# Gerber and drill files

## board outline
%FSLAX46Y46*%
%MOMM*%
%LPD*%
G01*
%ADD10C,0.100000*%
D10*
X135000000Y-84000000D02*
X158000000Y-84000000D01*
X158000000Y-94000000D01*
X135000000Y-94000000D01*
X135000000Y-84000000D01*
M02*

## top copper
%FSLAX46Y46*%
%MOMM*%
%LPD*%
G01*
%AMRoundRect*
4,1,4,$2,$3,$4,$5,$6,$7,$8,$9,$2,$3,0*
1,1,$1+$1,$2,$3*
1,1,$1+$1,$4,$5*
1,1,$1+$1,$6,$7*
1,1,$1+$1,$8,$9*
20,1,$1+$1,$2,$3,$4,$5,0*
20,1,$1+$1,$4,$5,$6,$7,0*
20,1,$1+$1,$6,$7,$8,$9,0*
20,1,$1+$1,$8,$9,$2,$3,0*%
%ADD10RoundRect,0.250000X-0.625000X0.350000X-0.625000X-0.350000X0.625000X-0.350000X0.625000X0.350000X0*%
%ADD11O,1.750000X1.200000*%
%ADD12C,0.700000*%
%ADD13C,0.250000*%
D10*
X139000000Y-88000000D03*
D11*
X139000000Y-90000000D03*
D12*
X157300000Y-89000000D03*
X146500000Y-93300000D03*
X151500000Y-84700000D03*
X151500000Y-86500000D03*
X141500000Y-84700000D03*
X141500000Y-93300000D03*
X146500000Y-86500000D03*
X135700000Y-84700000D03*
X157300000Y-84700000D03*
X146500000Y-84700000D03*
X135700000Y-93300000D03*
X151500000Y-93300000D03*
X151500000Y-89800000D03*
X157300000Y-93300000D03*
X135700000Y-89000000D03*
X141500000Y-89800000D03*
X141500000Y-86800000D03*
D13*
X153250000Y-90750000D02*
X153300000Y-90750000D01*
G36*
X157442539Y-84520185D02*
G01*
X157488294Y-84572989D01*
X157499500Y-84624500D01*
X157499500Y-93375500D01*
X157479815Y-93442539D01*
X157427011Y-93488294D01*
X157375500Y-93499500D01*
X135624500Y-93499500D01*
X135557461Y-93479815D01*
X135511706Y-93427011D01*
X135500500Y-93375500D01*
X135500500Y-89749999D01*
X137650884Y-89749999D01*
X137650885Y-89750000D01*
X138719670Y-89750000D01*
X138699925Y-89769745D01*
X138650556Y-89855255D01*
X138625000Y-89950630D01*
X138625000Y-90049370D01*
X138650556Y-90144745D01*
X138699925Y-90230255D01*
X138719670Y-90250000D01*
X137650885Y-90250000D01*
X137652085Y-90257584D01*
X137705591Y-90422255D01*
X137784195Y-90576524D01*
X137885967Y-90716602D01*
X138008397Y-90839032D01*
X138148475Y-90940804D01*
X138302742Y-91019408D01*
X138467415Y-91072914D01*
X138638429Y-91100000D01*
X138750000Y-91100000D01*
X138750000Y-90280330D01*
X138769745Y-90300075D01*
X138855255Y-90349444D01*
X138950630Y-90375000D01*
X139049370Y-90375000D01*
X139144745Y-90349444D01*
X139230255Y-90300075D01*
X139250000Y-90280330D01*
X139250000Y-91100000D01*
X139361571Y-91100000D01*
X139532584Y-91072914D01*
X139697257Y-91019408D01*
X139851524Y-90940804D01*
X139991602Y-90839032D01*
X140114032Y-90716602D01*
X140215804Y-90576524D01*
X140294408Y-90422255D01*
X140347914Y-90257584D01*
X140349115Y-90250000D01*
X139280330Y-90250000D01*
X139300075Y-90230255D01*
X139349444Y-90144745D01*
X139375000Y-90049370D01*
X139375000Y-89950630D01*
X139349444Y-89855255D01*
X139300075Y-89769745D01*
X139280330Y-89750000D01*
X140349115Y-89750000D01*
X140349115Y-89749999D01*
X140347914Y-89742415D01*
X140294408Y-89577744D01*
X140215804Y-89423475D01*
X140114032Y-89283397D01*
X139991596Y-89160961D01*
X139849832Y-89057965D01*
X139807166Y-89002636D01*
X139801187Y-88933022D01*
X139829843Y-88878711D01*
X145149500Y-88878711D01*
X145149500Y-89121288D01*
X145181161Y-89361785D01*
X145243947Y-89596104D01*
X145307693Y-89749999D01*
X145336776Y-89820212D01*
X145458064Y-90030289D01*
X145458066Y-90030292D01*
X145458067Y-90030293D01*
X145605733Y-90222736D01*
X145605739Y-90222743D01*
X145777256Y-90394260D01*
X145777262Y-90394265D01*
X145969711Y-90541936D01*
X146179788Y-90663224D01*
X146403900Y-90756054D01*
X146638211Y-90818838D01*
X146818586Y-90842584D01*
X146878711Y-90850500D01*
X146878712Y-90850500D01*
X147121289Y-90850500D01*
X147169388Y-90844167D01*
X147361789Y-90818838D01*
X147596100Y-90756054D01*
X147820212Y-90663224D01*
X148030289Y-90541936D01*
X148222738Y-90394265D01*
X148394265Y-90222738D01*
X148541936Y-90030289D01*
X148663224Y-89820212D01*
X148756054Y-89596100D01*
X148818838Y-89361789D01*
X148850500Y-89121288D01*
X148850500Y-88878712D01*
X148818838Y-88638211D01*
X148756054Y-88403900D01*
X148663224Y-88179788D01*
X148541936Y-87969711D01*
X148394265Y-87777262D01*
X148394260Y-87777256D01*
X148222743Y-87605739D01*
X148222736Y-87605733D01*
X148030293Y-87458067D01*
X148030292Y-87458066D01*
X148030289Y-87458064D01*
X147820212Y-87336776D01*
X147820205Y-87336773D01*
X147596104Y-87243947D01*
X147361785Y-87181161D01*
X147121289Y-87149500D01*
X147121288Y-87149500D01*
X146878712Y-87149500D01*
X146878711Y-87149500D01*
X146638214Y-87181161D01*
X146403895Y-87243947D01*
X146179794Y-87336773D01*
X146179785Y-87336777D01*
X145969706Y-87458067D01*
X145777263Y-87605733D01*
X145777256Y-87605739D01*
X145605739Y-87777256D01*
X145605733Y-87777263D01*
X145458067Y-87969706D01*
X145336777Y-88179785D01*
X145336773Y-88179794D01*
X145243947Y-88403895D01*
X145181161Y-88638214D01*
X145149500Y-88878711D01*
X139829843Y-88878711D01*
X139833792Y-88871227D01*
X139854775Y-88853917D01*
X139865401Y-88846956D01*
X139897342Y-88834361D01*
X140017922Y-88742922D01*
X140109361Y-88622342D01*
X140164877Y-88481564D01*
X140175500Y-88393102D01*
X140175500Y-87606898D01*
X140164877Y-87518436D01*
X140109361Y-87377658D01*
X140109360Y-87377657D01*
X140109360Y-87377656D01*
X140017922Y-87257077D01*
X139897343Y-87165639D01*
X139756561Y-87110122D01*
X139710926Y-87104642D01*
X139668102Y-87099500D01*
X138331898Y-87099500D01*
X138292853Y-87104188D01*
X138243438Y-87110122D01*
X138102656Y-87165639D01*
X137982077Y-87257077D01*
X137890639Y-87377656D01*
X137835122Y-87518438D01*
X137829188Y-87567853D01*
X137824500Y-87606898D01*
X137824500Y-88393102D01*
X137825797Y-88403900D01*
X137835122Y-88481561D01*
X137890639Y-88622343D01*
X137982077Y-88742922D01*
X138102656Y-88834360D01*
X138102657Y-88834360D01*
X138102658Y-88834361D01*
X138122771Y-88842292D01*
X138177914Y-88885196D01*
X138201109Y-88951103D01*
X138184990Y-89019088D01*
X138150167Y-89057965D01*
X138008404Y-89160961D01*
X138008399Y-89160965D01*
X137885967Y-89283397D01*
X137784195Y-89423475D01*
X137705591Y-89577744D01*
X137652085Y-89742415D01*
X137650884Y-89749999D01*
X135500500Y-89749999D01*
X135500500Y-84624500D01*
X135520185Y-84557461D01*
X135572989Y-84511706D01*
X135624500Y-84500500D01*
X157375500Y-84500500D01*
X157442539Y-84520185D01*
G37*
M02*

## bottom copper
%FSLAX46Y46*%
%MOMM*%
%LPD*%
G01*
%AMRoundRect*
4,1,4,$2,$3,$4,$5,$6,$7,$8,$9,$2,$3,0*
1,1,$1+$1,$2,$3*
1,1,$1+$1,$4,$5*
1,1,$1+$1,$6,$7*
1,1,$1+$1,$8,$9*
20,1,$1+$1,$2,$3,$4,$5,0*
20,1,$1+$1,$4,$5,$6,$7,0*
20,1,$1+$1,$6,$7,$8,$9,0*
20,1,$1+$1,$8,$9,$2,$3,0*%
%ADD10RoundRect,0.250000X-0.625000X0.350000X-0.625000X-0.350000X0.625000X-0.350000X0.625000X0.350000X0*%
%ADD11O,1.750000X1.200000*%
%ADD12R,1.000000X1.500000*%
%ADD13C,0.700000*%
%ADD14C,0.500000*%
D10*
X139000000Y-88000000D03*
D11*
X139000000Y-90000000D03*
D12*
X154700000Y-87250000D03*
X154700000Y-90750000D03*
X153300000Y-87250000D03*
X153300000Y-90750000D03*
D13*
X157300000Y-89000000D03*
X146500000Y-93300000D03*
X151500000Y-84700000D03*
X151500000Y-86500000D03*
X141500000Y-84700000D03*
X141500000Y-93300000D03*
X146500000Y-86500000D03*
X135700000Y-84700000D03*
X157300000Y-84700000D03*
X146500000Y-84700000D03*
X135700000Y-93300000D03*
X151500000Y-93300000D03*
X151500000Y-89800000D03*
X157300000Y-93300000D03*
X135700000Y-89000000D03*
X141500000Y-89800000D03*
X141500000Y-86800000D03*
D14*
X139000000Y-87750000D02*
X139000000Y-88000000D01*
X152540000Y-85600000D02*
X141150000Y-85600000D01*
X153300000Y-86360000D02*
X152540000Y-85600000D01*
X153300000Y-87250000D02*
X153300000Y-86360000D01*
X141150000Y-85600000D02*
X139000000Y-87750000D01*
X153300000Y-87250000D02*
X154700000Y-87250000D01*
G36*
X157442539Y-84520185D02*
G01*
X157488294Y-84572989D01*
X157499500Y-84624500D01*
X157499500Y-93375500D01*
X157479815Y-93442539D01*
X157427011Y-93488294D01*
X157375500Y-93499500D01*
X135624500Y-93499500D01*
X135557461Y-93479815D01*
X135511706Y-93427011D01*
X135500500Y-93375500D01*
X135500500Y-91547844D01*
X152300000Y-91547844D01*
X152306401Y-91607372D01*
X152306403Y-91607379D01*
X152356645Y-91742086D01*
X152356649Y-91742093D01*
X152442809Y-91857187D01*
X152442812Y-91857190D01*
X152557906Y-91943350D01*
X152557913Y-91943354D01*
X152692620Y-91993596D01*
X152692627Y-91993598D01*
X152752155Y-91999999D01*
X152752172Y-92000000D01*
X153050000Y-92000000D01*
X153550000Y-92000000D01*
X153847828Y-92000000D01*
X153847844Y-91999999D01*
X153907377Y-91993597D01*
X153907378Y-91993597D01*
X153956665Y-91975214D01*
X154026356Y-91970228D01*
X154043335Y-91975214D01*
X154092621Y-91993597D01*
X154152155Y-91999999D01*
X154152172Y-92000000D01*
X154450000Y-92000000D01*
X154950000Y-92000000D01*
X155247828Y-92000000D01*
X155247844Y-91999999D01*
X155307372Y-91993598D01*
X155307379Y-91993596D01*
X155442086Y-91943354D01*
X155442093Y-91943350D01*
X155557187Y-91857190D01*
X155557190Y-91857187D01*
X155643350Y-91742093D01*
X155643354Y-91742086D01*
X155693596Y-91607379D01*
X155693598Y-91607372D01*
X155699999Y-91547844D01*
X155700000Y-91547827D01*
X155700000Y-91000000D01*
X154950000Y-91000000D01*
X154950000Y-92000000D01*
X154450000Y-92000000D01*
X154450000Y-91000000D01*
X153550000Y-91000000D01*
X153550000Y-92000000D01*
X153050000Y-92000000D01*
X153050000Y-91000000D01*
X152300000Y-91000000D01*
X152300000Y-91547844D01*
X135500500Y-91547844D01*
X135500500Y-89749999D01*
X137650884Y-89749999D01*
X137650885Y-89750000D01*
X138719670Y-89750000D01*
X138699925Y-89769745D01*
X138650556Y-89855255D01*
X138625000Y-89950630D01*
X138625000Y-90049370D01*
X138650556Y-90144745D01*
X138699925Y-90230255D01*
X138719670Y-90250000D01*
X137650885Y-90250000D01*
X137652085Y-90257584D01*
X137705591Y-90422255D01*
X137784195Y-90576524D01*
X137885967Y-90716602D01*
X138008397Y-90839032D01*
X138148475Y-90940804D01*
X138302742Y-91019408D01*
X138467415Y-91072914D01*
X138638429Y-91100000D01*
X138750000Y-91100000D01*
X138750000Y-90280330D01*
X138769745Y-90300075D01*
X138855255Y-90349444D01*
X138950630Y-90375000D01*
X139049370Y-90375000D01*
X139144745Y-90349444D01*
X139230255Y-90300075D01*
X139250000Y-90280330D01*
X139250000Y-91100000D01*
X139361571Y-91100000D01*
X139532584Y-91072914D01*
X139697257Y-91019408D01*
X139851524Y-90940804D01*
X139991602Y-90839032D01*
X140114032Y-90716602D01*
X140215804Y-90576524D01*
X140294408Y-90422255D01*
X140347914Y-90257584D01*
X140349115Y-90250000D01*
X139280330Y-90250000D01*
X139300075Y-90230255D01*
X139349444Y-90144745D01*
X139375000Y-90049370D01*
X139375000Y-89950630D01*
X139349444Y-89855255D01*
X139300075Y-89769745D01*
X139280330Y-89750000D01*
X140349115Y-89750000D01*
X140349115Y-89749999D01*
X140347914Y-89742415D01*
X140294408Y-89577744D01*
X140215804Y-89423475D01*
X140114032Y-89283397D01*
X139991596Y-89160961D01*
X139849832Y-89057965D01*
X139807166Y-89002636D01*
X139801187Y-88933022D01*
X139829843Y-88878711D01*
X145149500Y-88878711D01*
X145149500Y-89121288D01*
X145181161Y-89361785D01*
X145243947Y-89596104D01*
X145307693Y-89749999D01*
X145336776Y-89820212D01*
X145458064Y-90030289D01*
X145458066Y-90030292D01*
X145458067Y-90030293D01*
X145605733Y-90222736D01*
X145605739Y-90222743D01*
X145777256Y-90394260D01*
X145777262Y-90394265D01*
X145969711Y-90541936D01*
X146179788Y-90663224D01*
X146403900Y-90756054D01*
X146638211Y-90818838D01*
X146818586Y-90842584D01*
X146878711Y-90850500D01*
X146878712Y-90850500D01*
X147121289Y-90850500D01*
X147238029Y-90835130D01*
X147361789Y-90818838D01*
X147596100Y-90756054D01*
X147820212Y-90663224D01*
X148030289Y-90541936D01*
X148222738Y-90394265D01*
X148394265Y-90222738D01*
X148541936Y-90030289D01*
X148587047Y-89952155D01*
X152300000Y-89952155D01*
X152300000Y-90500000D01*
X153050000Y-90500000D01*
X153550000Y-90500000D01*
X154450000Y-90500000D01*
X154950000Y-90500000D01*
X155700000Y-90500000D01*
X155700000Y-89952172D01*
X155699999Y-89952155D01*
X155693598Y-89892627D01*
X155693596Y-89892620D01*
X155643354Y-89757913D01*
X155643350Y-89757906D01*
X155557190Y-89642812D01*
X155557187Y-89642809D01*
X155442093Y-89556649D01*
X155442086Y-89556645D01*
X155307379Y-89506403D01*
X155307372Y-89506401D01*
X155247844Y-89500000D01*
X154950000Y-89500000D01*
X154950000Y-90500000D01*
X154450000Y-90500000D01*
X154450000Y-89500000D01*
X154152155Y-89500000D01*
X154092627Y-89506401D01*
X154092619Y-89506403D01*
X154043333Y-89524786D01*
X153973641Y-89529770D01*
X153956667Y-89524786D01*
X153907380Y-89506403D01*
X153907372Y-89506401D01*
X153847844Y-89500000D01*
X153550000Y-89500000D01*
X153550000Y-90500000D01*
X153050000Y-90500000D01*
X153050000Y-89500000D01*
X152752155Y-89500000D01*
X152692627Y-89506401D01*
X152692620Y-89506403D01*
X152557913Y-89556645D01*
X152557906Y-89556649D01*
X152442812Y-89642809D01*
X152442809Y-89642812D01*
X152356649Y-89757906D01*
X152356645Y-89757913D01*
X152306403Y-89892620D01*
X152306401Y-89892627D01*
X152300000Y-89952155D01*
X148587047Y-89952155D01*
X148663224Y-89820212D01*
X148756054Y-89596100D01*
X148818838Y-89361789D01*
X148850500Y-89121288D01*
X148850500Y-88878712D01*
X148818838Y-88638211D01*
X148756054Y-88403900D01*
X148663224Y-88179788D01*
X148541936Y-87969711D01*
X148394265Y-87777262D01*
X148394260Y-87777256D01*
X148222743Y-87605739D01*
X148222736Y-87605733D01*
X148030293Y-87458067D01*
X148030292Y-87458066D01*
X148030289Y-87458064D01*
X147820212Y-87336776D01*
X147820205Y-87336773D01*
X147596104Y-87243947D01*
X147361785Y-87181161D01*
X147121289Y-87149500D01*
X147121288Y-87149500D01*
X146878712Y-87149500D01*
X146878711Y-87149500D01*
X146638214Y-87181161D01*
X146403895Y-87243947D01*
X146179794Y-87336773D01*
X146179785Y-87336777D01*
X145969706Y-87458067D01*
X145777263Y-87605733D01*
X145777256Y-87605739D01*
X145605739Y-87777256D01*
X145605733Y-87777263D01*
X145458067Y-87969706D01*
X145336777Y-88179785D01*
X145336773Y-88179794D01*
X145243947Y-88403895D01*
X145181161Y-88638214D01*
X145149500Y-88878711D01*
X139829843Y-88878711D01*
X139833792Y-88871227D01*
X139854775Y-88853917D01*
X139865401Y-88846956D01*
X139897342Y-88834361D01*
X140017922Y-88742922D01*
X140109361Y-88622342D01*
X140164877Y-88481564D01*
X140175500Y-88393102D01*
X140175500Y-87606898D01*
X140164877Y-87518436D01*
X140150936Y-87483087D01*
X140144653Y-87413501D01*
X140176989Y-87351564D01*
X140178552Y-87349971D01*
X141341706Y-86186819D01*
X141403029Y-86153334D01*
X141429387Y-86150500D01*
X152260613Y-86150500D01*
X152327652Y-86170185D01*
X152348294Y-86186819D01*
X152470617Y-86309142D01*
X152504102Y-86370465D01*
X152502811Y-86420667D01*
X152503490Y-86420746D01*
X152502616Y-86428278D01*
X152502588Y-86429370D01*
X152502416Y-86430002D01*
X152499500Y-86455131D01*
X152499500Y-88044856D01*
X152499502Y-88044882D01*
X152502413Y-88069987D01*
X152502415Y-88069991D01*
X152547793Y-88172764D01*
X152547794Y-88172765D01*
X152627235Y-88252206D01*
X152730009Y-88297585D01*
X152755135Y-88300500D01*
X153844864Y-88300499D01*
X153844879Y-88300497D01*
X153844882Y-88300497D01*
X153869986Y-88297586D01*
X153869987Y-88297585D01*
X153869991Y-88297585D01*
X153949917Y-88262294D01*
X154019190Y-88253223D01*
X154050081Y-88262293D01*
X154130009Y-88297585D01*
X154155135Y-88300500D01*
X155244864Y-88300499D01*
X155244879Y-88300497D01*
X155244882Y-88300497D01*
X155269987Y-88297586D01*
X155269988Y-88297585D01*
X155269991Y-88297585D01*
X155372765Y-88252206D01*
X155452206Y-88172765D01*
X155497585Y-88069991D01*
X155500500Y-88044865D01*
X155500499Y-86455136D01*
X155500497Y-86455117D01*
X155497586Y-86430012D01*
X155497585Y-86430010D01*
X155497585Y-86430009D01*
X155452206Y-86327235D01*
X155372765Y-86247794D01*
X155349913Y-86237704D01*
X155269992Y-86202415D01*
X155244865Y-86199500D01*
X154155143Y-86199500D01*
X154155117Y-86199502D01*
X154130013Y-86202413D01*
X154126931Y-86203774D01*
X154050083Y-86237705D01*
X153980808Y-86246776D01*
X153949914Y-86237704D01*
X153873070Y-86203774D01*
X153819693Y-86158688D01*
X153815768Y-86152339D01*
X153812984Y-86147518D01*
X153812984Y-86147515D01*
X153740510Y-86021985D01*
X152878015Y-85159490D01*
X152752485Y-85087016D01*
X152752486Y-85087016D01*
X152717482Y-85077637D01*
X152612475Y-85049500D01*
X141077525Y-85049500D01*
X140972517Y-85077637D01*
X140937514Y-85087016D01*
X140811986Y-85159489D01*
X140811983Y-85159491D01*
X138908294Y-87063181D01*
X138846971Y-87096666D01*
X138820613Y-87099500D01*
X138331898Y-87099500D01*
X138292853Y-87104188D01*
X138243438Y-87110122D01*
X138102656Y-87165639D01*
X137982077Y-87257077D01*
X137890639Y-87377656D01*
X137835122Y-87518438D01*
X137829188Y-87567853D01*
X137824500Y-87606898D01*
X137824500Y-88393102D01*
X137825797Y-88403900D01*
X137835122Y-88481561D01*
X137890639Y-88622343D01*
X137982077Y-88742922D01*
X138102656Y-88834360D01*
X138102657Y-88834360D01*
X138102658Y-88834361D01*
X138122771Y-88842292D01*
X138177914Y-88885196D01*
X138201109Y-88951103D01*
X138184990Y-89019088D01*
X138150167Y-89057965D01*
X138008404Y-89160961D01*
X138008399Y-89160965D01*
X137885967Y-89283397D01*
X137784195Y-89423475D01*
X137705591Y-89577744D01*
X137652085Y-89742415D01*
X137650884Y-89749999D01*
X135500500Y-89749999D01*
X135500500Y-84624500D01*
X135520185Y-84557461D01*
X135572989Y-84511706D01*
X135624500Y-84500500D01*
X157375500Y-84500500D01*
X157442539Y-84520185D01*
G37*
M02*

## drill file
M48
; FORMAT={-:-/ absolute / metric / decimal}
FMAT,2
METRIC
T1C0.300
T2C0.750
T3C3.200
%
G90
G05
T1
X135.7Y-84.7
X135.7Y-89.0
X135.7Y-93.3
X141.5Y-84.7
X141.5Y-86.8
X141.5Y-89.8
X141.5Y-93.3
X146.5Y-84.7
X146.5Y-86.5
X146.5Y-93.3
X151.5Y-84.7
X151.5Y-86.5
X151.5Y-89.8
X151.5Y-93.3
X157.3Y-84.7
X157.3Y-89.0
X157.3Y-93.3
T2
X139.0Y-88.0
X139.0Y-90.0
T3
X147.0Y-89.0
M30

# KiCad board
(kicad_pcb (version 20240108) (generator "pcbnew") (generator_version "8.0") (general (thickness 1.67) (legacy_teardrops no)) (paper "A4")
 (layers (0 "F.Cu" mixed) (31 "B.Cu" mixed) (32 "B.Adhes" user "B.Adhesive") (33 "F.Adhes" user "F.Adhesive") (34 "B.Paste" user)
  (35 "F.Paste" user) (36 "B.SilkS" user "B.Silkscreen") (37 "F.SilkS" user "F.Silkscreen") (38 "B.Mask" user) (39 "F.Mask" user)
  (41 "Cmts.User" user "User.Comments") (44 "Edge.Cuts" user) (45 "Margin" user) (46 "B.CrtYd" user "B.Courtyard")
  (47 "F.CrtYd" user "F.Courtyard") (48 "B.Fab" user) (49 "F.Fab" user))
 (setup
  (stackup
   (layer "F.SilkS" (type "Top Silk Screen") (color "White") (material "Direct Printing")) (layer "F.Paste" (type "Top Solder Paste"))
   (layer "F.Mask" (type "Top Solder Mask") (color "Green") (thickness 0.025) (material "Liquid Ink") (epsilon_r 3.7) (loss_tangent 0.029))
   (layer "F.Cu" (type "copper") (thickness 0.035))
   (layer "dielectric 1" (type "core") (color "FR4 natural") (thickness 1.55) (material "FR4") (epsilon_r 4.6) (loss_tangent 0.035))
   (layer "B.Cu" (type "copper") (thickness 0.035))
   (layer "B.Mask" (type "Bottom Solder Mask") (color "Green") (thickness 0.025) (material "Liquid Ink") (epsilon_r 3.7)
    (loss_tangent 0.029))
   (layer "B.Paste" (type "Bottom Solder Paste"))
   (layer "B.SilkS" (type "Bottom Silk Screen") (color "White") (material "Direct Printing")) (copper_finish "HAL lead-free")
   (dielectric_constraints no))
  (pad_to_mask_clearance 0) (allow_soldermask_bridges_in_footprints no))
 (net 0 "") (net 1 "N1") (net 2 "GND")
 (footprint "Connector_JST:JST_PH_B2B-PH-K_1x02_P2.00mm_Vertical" (layer "F.Cu") (at 139 88 -90)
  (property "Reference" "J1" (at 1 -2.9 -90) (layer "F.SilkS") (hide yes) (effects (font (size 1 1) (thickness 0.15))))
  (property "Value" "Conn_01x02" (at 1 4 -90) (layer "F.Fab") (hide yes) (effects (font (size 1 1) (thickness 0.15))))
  (pad "1" thru_hole roundrect (at 0 0 270) (size 1.2 1.75) (drill 0.75) (layers "*.Cu" "*.Mask") (remove_unused_layers no)
   (roundrect_rratio 0.208333) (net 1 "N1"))
  (pad "2" thru_hole oval (at 2 0 270) (size 1.2 1.75) (drill 0.75) (layers "*.Cu" "*.Mask") (remove_unused_layers no) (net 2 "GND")))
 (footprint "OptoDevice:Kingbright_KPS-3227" (layer "B.Cu") (at 154 89 180)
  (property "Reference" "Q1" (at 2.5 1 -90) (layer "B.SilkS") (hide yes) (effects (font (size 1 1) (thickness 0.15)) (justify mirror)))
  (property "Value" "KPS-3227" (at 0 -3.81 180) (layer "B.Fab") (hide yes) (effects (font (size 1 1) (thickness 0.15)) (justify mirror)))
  (pad "1" smd rect (at -0.7 1.75 180) (size 1 1.5) (layers "B.Cu" "B.Paste" "B.Mask") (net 1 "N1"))
  (pad "2" smd rect (at -0.7 -1.75 180) (size 1 1.5) (layers "B.Cu" "B.Paste" "B.Mask") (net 2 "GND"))
  (pad "3" smd rect (at 0.7 1.75 180) (size 1 1.5) (layers "B.Cu" "B.Paste" "B.Mask") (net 1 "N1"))
  (pad "4" smd rect (at 0.7 -1.75 180) (size 1 1.5) (layers "B.Cu" "B.Paste" "B.Mask") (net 2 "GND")))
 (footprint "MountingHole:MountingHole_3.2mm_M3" (layer "B.Cu") (at 147 89 -90)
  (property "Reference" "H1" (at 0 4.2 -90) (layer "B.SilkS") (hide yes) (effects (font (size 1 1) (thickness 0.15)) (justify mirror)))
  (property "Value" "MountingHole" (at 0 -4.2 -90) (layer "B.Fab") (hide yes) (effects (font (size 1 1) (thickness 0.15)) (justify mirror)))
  (pad "" np_thru_hole circle (at 0 0 270) (size 3.2 3.2) (drill 3.2) (layers "*.Cu" "*.Mask")))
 (gr_rect (start 135 84) (end 158 94) (stroke (width 0.1) (type default)) (fill none) (layer "Edge.Cuts"))
 (segment (start 139 87.75) (end 139 88) (width 0.5) (layer "B.Cu") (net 1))
 (segment (start 152.54 85.6) (end 141.15 85.6) (width 0.5) (layer "B.Cu") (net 1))
 (segment (start 153.3 86.36) (end 152.54 85.6) (width 0.5) (layer "B.Cu") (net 1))
 (segment (start 153.3 87.25) (end 153.3 86.36) (width 0.5) (layer "B.Cu") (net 1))
 (segment (start 141.15 85.6) (end 139 87.75) (width 0.5) (layer "B.Cu") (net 1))
 (segment (start 153.3 87.25) (end 154.7 87.25) (width 0.5) (layer "B.Cu") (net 1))
 (segment (start 153.25 90.75) (end 153.3 90.75) (width 0.25) (layer "F.Cu") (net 2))
 (via (at 157.3 89) (size 0.7) (drill 0.3) (layers "F.Cu" "B.Cu") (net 2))
 (via (at 146.5 93.3) (size 0.7) (drill 0.3) (layers "F.Cu" "B.Cu") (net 2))
 (via (at 151.5 84.7) (size 0.7) (drill 0.3) (layers "F.Cu" "B.Cu") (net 2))
 (via (at 151.5 86.5) (size 0.7) (drill 0.3) (layers "F.Cu" "B.Cu") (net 2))
 (via (at 141.5 84.7) (size 0.7) (drill 0.3) (layers "F.Cu" "B.Cu") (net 2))
 (via (at 141.5 93.3) (size 0.7) (drill 0.3) (layers "F.Cu" "B.Cu") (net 2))
 (via (at 146.5 86.5) (size 0.7) (drill 0.3) (layers "F.Cu" "B.Cu") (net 2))
 (via (at 135.7 84.7) (size 0.7) (drill 0.3) (layers "F.Cu" "B.Cu") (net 2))
 (via (at 157.3 84.7) (size 0.7) (drill 0.3) (layers "F.Cu" "B.Cu") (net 2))
 (via (at 146.5 84.7) (size 0.7) (drill 0.3) (layers "F.Cu" "B.Cu") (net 2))
 (via (at 135.7 93.3) (size 0.7) (drill 0.3) (layers "F.Cu" "B.Cu") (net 2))
 (via (at 151.5 93.3) (size 0.7) (drill 0.3) (layers "F.Cu" "B.Cu") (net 2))
 (via (at 151.5 89.8) (size 0.7) (drill 0.3) (layers "F.Cu" "B.Cu") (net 2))
 (via (at 157.3 93.3) (size 0.7) (drill 0.3) (layers "F.Cu" "B.Cu") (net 2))
 (via (at 135.7 89) (size 0.7) (drill 0.3) (layers "F.Cu" "B.Cu") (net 2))
 (via (at 141.5 89.8) (size 0.7) (drill 0.3) (layers "F.Cu" "B.Cu") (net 2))
 (via (at 141.5 86.8) (size 0.7) (drill 0.3) (layers "F.Cu" "B.Cu") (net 2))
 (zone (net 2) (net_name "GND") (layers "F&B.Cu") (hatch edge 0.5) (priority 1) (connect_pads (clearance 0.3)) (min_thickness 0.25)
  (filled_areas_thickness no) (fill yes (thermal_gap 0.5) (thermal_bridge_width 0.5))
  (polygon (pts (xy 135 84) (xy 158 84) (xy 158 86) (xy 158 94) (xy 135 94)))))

